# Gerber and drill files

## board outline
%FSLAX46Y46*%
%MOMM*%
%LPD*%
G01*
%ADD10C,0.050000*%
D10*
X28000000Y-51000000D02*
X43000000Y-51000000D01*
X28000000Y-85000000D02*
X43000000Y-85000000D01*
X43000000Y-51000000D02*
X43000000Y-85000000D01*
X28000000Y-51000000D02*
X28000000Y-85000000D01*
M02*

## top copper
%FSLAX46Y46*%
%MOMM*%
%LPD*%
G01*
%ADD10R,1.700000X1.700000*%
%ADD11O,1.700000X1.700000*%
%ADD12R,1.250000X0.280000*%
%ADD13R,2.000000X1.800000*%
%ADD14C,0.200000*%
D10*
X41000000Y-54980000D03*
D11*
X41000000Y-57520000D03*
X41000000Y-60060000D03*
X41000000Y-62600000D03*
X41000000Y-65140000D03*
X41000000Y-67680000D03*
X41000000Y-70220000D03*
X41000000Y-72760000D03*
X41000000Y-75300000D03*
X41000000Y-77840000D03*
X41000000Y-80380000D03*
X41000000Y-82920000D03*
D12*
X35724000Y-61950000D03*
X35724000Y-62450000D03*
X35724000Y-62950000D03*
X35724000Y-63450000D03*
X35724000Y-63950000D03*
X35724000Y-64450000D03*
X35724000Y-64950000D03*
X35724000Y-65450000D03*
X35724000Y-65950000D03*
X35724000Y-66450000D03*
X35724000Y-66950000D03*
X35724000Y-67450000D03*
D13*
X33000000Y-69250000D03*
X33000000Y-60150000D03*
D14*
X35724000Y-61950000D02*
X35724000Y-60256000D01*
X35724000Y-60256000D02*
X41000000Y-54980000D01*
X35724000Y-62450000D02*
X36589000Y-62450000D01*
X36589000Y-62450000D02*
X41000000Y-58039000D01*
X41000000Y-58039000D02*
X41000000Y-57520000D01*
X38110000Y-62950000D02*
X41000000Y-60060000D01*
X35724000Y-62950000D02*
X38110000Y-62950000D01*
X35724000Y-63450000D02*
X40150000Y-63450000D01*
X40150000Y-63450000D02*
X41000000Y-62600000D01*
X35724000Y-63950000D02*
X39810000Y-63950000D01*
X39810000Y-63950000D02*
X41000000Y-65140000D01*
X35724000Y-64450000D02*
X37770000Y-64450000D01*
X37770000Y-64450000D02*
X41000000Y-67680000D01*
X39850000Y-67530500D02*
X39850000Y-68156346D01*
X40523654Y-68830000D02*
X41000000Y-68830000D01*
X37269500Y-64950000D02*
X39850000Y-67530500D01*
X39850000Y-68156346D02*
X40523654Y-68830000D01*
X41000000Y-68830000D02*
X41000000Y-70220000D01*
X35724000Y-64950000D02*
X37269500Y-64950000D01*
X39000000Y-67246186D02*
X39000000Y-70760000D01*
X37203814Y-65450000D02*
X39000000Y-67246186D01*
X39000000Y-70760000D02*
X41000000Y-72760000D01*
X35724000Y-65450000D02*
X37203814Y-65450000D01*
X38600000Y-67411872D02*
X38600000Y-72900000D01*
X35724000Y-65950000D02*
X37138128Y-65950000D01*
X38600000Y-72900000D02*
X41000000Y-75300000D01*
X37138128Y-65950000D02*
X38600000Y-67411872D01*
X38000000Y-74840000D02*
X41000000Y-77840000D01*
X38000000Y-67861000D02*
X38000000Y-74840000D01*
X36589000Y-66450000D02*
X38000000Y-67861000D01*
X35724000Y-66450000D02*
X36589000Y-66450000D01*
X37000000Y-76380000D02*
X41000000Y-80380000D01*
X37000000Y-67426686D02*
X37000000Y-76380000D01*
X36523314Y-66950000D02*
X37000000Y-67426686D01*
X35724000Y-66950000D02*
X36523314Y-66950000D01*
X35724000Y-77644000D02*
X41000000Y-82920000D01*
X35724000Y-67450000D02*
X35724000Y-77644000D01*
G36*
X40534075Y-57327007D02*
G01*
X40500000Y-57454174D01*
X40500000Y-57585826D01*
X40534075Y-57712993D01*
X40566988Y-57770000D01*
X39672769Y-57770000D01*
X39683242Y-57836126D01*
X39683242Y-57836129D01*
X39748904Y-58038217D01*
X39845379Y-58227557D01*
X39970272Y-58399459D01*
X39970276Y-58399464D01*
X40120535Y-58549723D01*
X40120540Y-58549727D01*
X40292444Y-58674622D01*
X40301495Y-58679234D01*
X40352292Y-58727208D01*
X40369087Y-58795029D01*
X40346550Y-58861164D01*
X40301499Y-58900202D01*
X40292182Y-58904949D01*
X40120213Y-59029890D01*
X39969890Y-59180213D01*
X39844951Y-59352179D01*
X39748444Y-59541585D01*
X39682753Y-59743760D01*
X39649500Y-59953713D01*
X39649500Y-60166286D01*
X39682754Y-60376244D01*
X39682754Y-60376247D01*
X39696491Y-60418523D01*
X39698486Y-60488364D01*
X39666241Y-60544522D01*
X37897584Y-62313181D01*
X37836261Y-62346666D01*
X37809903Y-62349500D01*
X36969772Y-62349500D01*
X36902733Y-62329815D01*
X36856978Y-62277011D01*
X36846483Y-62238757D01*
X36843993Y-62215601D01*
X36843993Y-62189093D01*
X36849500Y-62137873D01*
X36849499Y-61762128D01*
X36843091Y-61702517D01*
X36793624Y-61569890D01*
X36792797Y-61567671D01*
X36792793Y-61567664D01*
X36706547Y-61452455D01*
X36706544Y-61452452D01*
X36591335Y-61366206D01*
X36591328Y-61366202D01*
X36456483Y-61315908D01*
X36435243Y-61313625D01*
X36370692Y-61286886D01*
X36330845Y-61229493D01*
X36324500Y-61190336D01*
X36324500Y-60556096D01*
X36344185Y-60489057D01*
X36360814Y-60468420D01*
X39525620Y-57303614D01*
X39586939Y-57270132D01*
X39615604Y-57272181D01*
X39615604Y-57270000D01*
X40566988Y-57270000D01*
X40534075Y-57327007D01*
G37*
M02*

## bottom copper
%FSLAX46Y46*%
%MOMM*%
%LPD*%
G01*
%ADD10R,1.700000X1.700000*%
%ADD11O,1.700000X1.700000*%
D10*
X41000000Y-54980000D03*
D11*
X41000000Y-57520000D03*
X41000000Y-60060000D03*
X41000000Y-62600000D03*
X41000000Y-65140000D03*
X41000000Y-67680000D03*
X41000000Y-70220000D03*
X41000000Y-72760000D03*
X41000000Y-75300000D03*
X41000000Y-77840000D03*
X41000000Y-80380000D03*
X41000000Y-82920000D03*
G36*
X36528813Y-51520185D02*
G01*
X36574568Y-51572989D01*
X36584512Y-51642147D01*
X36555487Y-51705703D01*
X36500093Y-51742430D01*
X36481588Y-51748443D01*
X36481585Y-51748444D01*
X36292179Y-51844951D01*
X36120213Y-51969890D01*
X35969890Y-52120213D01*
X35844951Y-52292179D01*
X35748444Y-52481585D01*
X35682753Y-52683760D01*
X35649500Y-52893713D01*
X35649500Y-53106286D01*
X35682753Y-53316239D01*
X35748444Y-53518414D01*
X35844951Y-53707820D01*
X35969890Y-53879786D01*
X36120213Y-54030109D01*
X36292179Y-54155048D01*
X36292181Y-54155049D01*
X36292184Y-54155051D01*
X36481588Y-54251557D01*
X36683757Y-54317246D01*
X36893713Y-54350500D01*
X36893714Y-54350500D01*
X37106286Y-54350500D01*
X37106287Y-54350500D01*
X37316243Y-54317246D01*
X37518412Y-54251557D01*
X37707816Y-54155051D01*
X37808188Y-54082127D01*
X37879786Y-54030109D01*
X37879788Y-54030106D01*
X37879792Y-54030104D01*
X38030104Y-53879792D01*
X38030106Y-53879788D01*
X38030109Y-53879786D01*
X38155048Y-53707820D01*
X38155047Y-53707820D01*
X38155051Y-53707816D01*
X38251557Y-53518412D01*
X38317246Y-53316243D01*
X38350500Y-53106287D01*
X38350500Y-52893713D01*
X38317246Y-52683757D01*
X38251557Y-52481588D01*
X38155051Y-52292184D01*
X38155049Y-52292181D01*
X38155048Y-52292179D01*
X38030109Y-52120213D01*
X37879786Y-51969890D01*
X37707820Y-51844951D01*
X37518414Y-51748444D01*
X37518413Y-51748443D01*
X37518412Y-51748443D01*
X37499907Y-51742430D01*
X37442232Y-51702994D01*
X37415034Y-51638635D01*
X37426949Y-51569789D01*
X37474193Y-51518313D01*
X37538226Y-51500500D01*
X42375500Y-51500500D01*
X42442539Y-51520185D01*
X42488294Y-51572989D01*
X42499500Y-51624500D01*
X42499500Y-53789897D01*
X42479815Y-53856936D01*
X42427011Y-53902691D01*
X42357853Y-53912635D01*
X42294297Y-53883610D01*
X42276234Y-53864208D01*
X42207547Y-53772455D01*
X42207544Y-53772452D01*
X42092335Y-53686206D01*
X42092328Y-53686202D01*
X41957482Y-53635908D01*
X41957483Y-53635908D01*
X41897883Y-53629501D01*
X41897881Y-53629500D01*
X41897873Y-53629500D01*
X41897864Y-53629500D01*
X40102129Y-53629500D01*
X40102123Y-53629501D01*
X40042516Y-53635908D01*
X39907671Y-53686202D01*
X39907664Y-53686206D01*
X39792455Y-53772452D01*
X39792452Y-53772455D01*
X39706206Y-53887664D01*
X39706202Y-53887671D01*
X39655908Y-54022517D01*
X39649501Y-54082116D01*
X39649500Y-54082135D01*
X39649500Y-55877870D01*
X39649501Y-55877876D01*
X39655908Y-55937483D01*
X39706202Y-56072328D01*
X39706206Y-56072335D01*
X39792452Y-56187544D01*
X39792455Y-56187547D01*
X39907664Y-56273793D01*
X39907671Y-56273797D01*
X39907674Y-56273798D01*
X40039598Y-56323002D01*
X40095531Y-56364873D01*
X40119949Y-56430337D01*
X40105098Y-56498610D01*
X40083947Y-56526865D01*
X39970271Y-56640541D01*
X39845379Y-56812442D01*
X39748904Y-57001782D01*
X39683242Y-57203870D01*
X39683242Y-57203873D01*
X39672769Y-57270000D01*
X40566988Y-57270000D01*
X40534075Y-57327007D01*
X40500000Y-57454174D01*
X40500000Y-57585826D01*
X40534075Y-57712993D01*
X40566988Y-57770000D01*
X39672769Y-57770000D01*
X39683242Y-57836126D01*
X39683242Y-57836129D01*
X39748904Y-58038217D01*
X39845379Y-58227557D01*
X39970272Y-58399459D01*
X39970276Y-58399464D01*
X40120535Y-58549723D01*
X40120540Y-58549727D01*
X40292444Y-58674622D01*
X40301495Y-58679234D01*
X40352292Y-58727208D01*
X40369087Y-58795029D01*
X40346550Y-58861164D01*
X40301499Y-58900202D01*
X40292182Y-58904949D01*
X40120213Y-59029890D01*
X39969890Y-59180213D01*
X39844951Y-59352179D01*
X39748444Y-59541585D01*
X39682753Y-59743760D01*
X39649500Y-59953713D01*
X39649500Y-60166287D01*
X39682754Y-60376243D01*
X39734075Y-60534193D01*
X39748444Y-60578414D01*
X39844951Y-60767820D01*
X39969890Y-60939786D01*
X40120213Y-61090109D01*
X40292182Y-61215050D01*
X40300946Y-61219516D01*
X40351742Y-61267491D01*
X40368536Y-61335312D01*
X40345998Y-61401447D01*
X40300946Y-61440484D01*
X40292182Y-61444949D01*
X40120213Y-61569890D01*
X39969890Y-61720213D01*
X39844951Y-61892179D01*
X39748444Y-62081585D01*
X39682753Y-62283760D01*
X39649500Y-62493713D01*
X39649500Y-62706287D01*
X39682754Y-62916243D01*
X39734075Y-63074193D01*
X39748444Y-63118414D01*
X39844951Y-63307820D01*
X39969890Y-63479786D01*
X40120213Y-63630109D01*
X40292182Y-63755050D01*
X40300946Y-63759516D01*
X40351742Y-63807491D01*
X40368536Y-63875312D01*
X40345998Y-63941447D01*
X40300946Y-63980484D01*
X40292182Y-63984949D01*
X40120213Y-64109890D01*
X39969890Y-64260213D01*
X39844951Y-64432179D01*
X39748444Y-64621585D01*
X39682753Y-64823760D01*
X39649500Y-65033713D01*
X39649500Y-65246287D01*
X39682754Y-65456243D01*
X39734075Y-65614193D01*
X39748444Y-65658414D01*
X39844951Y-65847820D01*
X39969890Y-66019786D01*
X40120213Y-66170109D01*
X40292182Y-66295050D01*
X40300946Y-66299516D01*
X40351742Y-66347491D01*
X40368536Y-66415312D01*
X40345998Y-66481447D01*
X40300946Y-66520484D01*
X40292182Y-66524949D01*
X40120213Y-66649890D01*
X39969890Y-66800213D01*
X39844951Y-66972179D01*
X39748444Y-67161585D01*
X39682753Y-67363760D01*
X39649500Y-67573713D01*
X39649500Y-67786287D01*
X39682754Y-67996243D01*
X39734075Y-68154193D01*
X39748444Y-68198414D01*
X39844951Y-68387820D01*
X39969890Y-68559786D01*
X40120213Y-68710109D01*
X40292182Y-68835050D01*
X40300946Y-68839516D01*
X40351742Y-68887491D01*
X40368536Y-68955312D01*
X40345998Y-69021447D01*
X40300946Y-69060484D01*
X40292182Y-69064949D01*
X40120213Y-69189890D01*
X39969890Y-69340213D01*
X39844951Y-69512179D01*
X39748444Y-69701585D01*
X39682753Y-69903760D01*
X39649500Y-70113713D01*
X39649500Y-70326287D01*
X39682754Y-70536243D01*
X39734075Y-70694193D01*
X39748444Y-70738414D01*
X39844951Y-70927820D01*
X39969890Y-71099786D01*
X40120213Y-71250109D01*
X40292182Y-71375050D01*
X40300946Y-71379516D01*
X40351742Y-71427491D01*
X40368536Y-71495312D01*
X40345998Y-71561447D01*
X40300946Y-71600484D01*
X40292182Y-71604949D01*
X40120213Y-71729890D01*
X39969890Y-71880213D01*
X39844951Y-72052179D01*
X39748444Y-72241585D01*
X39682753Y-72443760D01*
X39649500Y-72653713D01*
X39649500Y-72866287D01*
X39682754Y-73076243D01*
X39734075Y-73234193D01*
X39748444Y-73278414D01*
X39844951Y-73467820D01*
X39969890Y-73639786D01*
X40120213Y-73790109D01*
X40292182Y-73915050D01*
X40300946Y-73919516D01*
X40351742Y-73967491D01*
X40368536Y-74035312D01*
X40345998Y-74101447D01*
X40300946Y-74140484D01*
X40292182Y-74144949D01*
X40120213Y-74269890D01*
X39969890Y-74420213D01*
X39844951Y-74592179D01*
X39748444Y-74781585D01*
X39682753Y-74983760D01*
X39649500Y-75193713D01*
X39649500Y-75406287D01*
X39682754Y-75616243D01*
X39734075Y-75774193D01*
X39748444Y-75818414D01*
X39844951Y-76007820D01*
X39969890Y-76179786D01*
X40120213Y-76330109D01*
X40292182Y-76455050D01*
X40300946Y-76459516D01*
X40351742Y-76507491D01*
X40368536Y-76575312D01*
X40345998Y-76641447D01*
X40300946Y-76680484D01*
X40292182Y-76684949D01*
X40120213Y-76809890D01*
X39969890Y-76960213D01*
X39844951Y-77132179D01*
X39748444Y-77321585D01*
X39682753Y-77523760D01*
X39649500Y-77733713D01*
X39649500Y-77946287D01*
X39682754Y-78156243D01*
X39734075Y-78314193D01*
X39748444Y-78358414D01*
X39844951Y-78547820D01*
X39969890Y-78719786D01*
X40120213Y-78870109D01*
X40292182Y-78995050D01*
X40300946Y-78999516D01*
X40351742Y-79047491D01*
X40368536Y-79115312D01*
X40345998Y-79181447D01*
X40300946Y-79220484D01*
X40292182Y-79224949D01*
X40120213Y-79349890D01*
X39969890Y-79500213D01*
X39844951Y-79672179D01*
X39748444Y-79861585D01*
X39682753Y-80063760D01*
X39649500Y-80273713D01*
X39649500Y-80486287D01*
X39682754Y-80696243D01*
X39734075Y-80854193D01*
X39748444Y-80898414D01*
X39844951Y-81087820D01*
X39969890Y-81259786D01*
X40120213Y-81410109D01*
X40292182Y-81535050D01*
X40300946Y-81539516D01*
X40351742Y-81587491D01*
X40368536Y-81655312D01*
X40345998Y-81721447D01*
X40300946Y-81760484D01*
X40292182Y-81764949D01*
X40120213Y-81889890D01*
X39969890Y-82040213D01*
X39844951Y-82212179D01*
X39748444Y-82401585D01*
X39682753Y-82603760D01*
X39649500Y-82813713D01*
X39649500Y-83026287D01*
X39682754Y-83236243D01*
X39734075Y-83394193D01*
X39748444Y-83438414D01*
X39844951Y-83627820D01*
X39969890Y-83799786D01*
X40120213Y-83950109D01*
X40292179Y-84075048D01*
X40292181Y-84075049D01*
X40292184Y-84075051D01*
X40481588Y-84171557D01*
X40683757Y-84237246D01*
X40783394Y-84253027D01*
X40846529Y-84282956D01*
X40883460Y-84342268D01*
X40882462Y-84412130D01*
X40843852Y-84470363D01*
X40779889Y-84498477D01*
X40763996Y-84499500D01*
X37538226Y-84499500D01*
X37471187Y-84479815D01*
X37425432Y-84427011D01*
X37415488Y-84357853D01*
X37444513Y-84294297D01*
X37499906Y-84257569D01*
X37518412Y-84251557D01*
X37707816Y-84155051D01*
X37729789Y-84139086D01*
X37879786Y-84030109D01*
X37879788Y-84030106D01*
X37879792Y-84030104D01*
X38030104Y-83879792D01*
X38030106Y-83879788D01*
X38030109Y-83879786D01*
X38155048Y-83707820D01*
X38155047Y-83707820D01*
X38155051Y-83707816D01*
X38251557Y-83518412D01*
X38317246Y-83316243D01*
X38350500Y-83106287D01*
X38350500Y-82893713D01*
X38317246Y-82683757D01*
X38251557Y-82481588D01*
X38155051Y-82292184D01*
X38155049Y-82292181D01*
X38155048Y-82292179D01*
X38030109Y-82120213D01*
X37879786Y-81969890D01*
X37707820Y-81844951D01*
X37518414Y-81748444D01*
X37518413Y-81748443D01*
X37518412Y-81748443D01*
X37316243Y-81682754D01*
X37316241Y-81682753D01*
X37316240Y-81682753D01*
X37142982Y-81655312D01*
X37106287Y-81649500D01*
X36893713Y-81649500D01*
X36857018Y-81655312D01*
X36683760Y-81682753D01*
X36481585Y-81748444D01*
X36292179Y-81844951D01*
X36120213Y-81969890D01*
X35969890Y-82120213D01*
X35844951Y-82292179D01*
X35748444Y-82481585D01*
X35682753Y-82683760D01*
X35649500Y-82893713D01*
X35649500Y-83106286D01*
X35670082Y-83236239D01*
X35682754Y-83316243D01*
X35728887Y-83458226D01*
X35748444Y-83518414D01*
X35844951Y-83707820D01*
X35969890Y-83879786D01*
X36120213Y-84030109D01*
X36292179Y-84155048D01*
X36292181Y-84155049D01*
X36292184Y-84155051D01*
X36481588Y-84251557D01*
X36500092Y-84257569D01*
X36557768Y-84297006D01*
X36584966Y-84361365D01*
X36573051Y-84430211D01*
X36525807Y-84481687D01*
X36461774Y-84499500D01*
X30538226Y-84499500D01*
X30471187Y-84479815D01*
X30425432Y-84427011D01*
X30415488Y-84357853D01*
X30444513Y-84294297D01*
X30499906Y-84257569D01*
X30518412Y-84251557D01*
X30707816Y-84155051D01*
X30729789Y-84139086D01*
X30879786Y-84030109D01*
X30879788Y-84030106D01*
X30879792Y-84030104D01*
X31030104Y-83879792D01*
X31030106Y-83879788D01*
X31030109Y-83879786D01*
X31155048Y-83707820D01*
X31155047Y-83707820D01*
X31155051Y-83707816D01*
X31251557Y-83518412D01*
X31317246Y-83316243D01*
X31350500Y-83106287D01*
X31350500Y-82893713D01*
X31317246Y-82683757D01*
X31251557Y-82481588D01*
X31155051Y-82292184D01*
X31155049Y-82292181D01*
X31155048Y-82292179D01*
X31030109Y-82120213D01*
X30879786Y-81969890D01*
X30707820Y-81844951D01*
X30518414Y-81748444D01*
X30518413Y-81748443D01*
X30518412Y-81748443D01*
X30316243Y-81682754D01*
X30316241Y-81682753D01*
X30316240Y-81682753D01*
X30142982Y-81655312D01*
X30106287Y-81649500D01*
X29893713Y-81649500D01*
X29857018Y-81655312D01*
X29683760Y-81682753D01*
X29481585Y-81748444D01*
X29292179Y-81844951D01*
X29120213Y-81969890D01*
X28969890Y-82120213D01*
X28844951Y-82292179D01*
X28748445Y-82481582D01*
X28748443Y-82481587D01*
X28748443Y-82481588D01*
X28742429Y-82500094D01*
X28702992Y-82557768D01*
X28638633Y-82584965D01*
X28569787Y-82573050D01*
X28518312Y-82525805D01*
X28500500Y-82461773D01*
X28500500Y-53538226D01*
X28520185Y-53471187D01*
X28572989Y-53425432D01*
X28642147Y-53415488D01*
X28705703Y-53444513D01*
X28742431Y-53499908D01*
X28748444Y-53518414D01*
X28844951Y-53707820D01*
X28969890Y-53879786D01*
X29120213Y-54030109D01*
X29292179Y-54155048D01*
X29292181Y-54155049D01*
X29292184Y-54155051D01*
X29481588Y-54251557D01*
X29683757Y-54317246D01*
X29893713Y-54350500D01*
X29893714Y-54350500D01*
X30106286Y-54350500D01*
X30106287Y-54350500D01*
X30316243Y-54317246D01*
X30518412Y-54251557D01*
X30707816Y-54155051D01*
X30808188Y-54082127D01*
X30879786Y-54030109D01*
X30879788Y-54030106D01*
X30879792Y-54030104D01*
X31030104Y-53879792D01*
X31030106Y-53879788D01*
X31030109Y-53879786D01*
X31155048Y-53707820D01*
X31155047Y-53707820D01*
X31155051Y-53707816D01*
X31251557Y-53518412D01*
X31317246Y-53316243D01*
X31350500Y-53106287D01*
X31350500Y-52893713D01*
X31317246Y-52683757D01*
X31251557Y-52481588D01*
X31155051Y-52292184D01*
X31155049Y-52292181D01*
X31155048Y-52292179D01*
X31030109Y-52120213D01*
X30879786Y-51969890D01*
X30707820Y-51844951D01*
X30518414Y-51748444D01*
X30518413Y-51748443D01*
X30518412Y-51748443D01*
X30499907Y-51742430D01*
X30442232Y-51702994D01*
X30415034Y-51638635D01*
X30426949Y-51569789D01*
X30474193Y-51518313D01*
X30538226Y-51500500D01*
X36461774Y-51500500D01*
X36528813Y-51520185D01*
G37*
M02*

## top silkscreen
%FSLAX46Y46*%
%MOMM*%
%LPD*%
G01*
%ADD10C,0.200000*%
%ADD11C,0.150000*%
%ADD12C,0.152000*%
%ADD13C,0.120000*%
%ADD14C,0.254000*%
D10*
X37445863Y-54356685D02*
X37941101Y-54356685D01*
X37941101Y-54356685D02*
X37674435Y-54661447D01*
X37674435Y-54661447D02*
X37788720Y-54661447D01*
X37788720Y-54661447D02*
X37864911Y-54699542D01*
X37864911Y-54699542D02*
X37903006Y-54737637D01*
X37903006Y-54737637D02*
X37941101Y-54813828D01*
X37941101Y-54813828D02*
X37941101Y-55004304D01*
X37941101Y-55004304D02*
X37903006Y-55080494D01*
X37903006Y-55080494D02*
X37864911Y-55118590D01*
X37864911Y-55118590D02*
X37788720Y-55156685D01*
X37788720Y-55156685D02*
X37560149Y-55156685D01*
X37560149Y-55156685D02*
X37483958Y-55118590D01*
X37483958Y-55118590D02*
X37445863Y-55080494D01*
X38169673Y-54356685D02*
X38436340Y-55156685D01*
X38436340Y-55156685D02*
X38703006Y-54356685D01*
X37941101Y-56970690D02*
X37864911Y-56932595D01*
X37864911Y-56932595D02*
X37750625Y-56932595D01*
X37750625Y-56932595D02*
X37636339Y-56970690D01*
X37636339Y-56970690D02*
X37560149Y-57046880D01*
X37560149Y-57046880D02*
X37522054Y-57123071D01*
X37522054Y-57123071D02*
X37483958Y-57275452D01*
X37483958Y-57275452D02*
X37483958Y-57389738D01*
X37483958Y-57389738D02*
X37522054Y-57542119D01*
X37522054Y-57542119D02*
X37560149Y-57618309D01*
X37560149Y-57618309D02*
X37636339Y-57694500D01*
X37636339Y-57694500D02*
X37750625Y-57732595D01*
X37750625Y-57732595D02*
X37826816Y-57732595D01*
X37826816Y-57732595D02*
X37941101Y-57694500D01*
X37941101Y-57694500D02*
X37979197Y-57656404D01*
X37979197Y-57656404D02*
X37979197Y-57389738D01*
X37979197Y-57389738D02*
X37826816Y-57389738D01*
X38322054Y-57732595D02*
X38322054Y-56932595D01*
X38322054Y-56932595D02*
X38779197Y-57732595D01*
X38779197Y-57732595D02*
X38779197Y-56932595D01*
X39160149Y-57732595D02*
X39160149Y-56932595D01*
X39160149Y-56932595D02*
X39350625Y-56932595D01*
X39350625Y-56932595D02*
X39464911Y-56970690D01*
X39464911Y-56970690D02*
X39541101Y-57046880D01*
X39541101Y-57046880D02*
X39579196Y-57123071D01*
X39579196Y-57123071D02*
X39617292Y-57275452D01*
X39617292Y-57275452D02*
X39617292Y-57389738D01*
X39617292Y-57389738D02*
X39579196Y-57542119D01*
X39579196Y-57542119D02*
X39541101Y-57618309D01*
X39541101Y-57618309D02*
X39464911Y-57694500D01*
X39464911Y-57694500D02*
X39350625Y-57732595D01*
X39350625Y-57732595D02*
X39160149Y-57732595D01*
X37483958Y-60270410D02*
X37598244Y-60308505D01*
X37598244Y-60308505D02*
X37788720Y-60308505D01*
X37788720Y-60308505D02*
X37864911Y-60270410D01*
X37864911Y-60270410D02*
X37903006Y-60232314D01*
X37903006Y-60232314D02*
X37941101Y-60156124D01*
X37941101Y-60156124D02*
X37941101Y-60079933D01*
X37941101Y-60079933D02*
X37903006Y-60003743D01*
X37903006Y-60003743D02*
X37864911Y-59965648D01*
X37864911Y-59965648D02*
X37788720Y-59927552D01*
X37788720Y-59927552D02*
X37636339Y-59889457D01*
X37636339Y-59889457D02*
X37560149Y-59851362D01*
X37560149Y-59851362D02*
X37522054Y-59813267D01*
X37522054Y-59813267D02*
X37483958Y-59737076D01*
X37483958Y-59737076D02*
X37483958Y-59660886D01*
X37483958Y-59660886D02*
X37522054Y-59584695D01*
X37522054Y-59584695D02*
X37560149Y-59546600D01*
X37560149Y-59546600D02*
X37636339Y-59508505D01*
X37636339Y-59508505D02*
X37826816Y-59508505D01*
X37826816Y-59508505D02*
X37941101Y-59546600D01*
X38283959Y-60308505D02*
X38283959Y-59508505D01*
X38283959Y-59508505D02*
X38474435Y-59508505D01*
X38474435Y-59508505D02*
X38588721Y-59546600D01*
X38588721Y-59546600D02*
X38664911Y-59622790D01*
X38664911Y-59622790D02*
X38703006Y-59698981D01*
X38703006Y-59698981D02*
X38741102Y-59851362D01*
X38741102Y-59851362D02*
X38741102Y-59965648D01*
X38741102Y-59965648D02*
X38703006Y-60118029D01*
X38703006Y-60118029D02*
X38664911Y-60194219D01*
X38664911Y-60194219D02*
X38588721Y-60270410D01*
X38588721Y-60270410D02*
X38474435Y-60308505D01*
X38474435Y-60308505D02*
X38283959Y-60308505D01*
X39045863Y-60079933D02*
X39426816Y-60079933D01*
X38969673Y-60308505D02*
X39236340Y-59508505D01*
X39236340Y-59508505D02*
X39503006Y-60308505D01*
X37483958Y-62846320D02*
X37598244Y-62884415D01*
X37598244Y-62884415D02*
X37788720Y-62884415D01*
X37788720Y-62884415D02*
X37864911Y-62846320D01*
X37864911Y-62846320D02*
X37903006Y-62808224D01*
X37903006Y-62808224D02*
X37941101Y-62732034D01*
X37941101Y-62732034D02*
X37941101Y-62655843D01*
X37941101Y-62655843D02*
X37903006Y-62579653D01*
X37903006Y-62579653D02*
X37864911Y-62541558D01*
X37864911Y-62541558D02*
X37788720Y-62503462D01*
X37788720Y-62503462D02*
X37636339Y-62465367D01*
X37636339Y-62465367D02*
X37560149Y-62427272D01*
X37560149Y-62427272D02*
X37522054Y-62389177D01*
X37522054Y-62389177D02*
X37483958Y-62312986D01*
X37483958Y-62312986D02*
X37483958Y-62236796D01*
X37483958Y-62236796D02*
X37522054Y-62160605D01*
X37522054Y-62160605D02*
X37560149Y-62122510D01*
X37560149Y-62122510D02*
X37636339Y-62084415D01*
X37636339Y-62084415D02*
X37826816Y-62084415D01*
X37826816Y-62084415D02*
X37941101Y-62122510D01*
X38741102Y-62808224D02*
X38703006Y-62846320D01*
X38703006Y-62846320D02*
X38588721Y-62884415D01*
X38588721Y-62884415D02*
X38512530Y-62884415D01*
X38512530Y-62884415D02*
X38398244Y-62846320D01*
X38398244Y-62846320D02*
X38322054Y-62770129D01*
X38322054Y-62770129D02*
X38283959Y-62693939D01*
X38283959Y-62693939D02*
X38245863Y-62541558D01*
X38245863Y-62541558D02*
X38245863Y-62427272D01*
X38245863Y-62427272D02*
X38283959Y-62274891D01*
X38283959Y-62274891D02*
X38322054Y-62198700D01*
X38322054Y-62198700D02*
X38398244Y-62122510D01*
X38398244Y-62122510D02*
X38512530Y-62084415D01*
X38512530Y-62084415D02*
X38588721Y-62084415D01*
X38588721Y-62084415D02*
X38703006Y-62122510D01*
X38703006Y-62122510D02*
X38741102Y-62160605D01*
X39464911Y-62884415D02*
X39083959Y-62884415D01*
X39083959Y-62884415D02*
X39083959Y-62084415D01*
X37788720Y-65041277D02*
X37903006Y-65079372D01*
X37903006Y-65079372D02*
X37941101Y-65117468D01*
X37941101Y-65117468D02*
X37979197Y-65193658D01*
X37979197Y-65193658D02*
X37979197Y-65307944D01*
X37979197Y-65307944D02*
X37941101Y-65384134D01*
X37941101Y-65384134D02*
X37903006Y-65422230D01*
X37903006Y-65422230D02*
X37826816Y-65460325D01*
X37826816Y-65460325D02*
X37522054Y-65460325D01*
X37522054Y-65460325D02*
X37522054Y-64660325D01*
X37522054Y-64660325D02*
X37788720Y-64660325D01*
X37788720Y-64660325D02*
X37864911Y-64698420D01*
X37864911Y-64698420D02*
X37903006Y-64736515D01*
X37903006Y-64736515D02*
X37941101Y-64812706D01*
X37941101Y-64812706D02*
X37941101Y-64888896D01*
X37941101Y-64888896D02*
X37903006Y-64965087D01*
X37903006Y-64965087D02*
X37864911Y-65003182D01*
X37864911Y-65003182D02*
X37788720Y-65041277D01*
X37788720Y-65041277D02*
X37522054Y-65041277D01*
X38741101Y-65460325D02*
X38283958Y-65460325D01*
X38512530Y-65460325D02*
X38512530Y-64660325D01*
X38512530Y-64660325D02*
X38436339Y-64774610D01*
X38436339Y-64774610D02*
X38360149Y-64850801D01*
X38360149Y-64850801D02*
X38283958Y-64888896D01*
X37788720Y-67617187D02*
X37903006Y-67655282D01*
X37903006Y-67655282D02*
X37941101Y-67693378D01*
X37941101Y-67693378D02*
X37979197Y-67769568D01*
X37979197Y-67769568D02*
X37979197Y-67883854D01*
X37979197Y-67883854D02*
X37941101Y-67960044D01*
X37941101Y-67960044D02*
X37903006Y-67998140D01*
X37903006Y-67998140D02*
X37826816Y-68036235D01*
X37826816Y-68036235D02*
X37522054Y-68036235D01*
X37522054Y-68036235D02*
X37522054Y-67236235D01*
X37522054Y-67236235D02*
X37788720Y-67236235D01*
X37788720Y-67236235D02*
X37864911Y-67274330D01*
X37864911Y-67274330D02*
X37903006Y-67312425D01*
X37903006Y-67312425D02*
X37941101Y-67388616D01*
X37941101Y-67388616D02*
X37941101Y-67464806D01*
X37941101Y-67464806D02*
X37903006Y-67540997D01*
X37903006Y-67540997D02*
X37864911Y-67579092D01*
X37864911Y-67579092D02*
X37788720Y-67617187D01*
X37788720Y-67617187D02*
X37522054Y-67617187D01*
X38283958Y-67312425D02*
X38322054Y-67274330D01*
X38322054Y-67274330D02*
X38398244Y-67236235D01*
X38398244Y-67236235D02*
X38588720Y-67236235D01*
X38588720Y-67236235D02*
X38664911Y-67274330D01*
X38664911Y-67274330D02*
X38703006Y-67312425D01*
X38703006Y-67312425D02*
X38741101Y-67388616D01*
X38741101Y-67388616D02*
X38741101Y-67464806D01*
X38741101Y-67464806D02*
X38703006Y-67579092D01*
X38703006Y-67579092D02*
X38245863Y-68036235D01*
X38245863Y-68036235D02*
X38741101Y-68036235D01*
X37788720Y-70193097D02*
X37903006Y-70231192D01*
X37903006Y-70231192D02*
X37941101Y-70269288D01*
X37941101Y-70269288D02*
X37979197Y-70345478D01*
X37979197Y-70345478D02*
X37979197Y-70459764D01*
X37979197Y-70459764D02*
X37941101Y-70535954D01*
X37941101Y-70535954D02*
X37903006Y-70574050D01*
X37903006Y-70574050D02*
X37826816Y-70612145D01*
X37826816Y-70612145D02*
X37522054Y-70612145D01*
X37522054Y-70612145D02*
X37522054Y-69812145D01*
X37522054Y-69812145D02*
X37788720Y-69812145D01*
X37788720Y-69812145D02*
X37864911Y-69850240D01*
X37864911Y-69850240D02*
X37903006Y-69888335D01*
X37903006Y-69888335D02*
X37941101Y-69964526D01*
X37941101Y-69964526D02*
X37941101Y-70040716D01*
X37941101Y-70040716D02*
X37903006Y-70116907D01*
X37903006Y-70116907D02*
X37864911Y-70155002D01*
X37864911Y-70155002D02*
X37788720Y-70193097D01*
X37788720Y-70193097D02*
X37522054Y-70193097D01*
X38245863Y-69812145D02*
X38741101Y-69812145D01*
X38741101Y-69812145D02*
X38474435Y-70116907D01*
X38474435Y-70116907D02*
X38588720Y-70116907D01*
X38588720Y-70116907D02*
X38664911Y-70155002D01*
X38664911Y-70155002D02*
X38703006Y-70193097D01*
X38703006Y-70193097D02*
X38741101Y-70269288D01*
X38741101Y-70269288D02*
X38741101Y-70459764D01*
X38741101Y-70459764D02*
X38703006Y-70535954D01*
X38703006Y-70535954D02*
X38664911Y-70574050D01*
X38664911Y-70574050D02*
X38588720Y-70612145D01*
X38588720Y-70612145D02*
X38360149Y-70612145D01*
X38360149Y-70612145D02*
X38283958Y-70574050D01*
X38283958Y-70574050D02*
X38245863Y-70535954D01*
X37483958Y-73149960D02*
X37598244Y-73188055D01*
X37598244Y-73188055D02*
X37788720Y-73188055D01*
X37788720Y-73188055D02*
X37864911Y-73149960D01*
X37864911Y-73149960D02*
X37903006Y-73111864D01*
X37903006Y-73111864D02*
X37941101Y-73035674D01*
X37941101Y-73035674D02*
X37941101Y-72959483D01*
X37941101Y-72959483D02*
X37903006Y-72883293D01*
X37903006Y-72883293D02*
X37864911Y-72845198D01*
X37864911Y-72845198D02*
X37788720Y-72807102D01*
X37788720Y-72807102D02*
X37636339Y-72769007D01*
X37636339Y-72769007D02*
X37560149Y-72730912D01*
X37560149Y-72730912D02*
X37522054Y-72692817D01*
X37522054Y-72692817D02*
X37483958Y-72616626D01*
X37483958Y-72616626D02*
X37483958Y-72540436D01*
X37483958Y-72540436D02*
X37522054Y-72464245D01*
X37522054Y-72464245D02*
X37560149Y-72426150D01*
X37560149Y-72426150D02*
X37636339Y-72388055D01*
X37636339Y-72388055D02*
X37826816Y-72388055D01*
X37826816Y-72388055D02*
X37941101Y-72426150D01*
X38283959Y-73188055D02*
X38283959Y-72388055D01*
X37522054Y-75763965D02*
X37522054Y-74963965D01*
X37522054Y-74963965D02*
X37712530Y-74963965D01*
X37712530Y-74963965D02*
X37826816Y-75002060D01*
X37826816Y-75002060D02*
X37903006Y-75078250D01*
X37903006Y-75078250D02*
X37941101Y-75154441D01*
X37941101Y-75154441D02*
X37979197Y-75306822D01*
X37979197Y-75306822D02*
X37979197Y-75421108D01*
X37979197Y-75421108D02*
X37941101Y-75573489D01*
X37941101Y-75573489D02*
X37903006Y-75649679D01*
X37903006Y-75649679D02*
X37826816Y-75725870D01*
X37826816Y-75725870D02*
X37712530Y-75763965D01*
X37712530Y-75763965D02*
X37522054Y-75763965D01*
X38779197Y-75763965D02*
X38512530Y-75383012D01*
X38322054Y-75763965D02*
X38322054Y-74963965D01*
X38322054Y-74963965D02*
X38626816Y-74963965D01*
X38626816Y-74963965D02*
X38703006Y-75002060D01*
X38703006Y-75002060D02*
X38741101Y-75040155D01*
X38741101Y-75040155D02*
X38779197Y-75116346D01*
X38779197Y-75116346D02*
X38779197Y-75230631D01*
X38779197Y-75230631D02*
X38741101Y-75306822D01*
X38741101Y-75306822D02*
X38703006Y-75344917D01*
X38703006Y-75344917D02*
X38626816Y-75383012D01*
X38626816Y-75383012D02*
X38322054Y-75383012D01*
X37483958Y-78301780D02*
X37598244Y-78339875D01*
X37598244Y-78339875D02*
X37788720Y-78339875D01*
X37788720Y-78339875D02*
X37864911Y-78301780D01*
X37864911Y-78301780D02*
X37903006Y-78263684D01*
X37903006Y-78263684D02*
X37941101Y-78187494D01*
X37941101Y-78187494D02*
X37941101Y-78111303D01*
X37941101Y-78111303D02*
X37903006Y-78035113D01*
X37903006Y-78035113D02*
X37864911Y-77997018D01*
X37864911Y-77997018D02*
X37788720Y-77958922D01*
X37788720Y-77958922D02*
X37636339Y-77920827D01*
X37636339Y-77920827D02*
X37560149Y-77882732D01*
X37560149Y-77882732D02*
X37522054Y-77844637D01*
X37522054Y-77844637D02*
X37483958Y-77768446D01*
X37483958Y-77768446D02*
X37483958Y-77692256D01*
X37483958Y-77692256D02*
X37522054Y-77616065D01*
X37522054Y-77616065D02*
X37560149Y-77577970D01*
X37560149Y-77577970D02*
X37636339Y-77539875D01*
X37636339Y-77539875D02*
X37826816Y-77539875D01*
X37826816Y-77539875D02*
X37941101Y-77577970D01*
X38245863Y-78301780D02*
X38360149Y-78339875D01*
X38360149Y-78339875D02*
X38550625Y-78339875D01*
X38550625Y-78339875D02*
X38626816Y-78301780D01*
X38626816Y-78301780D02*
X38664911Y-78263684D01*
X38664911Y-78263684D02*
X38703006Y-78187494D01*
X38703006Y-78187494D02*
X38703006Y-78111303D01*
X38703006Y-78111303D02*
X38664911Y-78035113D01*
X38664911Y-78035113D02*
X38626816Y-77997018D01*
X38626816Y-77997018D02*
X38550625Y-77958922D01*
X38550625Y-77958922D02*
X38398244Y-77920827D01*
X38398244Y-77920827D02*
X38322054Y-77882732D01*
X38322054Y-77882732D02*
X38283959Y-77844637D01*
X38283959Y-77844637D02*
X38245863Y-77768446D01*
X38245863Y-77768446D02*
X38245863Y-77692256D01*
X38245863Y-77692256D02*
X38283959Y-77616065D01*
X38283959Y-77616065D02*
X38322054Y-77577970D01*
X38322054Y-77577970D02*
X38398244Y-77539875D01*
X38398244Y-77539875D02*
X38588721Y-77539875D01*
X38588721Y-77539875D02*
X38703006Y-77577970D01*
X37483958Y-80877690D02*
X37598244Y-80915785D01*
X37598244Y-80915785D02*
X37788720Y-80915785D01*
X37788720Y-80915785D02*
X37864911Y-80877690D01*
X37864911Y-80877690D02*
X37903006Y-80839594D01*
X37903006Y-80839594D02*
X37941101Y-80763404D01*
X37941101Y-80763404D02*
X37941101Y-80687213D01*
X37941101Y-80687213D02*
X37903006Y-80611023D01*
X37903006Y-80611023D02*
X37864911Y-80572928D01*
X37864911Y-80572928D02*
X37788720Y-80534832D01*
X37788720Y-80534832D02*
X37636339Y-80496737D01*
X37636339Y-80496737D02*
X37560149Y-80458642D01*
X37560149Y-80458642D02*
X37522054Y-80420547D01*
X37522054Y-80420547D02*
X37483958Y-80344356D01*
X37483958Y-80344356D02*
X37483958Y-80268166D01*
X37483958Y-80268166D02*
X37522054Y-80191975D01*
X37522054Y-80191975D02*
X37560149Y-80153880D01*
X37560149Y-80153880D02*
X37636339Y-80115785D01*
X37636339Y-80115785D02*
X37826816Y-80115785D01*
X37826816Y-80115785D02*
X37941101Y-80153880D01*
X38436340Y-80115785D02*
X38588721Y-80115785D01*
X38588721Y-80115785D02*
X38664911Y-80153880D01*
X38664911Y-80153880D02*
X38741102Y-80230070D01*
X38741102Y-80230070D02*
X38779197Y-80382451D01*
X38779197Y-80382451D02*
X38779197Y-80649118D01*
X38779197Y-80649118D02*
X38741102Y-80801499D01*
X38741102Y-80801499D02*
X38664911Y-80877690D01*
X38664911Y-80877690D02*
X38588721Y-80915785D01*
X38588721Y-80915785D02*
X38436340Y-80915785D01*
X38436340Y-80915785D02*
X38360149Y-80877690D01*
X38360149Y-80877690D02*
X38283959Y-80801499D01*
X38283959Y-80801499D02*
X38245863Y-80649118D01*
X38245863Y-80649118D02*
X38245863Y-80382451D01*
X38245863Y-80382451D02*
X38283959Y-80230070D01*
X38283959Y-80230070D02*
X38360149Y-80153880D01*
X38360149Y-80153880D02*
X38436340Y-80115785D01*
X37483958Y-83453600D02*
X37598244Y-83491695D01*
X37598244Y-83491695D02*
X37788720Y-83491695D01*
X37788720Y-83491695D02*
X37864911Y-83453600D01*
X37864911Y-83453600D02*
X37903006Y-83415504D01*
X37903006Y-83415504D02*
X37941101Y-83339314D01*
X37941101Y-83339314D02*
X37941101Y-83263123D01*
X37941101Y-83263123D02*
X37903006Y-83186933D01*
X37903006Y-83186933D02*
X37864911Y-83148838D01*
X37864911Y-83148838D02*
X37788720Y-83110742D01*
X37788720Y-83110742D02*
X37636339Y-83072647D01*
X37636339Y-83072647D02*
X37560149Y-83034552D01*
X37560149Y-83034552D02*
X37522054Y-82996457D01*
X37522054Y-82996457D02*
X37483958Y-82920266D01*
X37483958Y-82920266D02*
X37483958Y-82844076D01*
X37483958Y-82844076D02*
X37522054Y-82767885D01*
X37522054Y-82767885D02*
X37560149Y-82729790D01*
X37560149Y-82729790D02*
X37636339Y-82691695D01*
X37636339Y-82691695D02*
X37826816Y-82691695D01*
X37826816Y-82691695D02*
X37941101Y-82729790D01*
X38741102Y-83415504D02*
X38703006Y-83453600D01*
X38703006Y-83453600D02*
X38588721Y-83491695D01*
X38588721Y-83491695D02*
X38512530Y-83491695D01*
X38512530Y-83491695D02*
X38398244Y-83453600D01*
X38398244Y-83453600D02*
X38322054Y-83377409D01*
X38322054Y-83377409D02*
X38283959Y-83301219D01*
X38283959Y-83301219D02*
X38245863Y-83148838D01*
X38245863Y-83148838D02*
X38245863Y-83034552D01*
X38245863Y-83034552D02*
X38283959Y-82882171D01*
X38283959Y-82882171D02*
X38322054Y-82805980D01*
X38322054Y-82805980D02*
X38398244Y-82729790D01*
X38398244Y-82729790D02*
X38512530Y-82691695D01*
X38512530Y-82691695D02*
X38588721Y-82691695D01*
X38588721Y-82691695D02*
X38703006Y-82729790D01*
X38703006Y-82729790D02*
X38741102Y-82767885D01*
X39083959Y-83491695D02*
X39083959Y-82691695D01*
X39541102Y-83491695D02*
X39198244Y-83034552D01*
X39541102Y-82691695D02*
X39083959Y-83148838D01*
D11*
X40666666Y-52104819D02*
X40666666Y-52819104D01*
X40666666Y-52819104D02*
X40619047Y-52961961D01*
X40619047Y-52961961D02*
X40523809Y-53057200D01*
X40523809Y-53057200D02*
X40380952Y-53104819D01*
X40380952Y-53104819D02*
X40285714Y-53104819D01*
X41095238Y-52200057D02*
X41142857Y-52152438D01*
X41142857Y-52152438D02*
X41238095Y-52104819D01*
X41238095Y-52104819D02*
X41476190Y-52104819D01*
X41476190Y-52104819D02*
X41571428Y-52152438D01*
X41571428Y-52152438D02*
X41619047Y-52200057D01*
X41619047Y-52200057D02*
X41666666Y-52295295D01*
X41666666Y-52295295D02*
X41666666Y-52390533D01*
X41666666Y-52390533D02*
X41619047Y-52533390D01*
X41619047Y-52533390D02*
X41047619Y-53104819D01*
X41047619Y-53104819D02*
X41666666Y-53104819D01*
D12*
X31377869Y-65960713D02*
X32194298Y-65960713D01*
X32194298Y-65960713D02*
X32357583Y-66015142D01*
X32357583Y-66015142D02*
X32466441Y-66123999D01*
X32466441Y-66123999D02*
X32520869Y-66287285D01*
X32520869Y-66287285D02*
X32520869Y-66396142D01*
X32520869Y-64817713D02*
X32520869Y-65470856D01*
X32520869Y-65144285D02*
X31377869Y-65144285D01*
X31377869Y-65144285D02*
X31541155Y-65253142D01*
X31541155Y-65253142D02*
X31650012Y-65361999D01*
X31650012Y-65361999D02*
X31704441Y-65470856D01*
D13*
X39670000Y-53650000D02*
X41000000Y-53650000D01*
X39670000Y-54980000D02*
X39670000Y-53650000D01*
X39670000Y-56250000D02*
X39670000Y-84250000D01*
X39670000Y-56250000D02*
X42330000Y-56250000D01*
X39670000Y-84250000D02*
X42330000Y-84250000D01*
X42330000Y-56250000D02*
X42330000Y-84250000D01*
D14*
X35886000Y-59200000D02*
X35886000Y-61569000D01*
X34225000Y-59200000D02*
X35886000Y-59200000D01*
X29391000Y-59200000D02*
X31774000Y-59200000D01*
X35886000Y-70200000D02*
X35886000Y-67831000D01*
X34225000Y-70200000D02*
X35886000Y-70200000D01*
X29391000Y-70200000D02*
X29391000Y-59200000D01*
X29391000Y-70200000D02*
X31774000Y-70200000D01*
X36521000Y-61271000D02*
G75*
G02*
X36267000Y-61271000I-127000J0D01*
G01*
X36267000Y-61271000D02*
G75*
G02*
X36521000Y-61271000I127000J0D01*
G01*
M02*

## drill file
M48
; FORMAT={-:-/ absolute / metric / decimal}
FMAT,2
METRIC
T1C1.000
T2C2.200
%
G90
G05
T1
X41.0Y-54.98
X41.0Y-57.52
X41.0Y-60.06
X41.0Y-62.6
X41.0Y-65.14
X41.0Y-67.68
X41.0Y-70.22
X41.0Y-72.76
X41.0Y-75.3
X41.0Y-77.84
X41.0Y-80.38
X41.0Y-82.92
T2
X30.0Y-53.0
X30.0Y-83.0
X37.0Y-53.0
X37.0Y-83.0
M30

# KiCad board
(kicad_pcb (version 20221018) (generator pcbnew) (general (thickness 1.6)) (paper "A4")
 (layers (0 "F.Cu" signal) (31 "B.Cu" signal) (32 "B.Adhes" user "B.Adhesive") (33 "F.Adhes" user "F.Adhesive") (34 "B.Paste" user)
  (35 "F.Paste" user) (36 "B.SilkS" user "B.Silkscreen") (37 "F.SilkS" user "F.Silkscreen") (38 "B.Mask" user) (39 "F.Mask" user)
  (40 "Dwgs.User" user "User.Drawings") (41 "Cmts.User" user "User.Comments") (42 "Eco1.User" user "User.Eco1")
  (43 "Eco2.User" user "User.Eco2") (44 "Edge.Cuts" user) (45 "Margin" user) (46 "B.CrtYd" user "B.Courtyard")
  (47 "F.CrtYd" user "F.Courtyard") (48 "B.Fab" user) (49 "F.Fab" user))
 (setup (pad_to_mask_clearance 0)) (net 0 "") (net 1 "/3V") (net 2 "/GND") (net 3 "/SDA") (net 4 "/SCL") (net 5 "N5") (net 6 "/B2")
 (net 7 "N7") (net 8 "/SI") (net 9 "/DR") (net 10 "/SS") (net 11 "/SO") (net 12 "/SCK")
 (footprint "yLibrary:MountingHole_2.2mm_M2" (layer "F.Cu") (at 37 53)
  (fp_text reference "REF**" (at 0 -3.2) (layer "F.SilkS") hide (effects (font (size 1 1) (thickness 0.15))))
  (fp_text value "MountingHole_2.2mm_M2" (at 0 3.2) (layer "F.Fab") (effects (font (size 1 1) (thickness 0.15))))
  (pad "" np_thru_hole circle (at 0 0) (size 2.2 2.2) (drill 2.2) (layers "*.Cu" "*.Mask")))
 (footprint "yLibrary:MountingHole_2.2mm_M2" (layer "F.Cu") (at 30 83)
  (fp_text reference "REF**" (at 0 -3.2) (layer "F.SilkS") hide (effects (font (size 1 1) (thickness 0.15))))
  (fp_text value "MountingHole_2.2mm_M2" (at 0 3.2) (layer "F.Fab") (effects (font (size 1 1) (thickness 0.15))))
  (pad "" np_thru_hole circle (at 0 0) (size 2.2 2.2) (drill 2.2) (layers "*.Cu" "*.Mask")))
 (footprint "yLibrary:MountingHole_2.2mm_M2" (layer "F.Cu") (at 30 53)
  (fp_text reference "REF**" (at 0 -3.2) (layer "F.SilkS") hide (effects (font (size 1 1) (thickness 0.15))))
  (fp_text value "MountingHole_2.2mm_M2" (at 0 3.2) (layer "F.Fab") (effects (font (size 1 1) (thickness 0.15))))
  (pad "" np_thru_hole circle (at 0 0) (size 2.2 2.2) (drill 2.2) (layers "*.Cu" "*.Mask")))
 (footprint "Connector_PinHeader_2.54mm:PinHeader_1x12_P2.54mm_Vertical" (layer "F.Cu") (at 41 54.98)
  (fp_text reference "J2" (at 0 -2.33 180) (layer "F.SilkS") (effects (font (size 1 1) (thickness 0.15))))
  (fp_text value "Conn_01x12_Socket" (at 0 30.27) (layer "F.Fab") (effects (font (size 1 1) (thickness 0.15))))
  (fp_line (start -1.33 -1.33) (end 0 -1.33) (stroke (width 0.12) (type solid)) (layer "F.SilkS"))
  (fp_line (start -1.33 0) (end -1.33 -1.33) (stroke (width 0.12) (type solid)) (layer "F.SilkS"))
  (fp_line (start -1.33 1.27) (end -1.33 29.27) (stroke (width 0.12) (type solid)) (layer "F.SilkS"))
  (fp_line (start -1.33 1.27) (end 1.33 1.27) (stroke (width 0.12) (type solid)) (layer "F.SilkS"))
  (fp_line (start -1.33 29.27) (end 1.33 29.27) (stroke (width 0.12) (type solid)) (layer "F.SilkS"))
  (fp_line (start 1.33 1.27) (end 1.33 29.27) (stroke (width 0.12) (type solid)) (layer "F.SilkS"))
  (pad "1" thru_hole rect (at 0 0) (size 1.7 1.7) (drill 1) (layers "*.Cu" "*.Mask") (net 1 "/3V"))
  (pad "2" thru_hole oval (at 0 2.54) (size 1.7 1.7) (drill 1) (layers "*.Cu" "*.Mask") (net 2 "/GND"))
  (pad "3" thru_hole oval (at 0 5.08) (size 1.7 1.7) (drill 1) (layers "*.Cu" "*.Mask") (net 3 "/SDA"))
  (pad "4" thru_hole oval (at 0 7.62) (size 1.7 1.7) (drill 1) (layers "*.Cu" "*.Mask") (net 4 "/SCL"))
  (pad "5" thru_hole oval (at 0 10.16) (size 1.7 1.7) (drill 1) (layers "*.Cu" "*.Mask") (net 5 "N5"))
  (pad "6" thru_hole oval (at 0 12.7) (size 1.7 1.7) (drill 1) (layers "*.Cu" "*.Mask") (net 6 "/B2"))
  (pad "7" thru_hole oval (at 0 15.24) (size 1.7 1.7) (drill 1) (layers "*.Cu" "*.Mask") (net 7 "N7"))
  (pad "8" thru_hole oval (at 0 17.78) (size 1.7 1.7) (drill 1) (layers "*.Cu" "*.Mask") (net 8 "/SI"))
  (pad "9" thru_hole oval (at 0 20.32) (size 1.7 1.7) (drill 1) (layers "*.Cu" "*.Mask") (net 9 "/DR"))
  (pad "10" thru_hole oval (at 0 22.86) (size 1.7 1.7) (drill 1) (layers "*.Cu" "*.Mask") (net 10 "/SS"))
  (pad "11" thru_hole oval (at 0 25.4) (size 1.7 1.7) (drill 1) (layers "*.Cu" "*.Mask") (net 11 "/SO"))
  (pad "12" thru_hole oval (at 0 27.94) (size 1.7 1.7) (drill 1) (layers "*.Cu" "*.Mask") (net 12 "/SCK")))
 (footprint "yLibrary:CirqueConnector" (layer "F.Cu") (at 34.362 64.7 -90)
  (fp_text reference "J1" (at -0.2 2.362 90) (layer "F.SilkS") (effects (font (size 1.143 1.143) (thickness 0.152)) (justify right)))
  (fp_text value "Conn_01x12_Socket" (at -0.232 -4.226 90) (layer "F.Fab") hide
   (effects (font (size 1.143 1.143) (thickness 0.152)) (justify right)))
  (fp_line (start -5.5 -1.524) (end -3.131 -1.524) (stroke (width 0.254) (type solid)) (layer "F.SilkS"))
  (fp_line (start -5.5 0.137) (end -5.5 -1.524) (stroke (width 0.254) (type solid)) (layer "F.SilkS"))
  (fp_line (start -5.5 4.971) (end -5.5 2.588) (stroke (width 0.254) (type solid)) (layer "F.SilkS"))
  (fp_line (start 5.5 -1.524) (end 3.131 -1.524) (stroke (width 0.254) (type solid)) (layer "F.SilkS"))
  (fp_line (start 5.5 0.137) (end 5.5 -1.524) (stroke (width 0.254) (type solid)) (layer "F.SilkS"))
  (fp_line (start 5.5 4.971) (end -5.5 4.971) (stroke (width 0.254) (type solid)) (layer "F.SilkS"))
  (fp_line (start 5.5 4.971) (end 5.5 2.588) (stroke (width 0.254) (type solid)) (layer "F.SilkS"))
  (fp_circle (center -3.429 -2.032) (end -3.302 -2.032) (stroke (width 0.254) (type solid)) (fill none) (layer "F.SilkS"))
  (pad "1" smd rect (at -2.75 -1.362 270) (size 0.28 1.25) (layers "F.Cu" "F.Paste" "F.Mask") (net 1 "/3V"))
  (pad "2" smd rect (at -2.25 -1.362 270) (size 0.28 1.25) (layers "F.Cu" "F.Paste" "F.Mask") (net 2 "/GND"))
  (pad "3" smd rect (at -1.75 -1.362 270) (size 0.28 1.25) (layers "F.Cu" "F.Paste" "F.Mask") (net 3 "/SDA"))
  (pad "4" smd rect (at -1.25 -1.362 270) (size 0.28 1.25) (layers "F.Cu" "F.Paste" "F.Mask") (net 4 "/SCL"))
  (pad "5" smd rect (at -0.75 -1.362 270) (size 0.28 1.25) (layers "F.Cu" "F.Paste" "F.Mask") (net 5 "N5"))
  (pad "6" smd rect (at -0.25 -1.362 270) (size 0.28 1.25) (layers "F.Cu" "F.Paste" "F.Mask") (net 6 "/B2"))
  (pad "7" smd rect (at 0.25 -1.362 270) (size 0.28 1.25) (layers "F.Cu" "F.Paste" "F.Mask") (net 7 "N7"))
  (pad "8" smd rect (at 0.75 -1.362 270) (size 0.28 1.25) (layers "F.Cu" "F.Paste" "F.Mask") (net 8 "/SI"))
  (pad "9" smd rect (at 1.25 -1.362 270) (size 0.28 1.25) (layers "F.Cu" "F.Paste" "F.Mask") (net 9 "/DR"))
  (pad "10" smd rect (at 1.75 -1.362 270) (size 0.28 1.25) (layers "F.Cu" "F.Paste" "F.Mask") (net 10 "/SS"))
  (pad "11" smd rect (at 2.25 -1.362 270) (size 0.28 1.25) (layers "F.Cu" "F.Paste" "F.Mask") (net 11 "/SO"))
  (pad "12" smd rect (at 2.75 -1.362 270) (size 0.28 1.25) (layers "F.Cu" "F.Paste" "F.Mask") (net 12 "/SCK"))
  (pad "13" smd rect (at 4.55 1.362 270) (size 1.8 2) (layers "F.Cu" "F.Paste" "F.Mask"))
  (pad "14" smd rect (at -4.55 1.362 270) (size 1.8 2) (layers "F.Cu" "F.Paste" "F.Mask")))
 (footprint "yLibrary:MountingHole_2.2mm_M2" (layer "F.Cu") (at 37 83)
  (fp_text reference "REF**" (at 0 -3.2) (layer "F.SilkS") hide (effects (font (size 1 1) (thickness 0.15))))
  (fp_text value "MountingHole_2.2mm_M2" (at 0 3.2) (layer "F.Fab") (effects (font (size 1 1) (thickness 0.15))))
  (pad "" np_thru_hole circle (at 0 0) (size 2.2 2.2) (drill 2.2) (layers "*.Cu" "*.Mask")))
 (gr_line (start 28 51) (end 43 51) (stroke (width 0.05) (type default)) (layer "Edge.Cuts"))
 (gr_line (start 28 85) (end 43 85) (stroke (width 0.05) (type default)) (layer "Edge.Cuts"))
 (gr_line (start 43 51) (end 43 85) (stroke (width 0.05) (type default)) (layer "Edge.Cuts"))
 (gr_line (start 28 51) (end 28 85) (stroke (width 0.05) (type default)) (layer "Edge.Cuts"))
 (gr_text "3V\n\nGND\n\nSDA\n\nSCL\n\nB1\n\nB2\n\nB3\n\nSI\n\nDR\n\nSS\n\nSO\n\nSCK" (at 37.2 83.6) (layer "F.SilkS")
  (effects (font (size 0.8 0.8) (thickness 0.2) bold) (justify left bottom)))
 (segment (start 35.724 61.95) (end 35.724 60.256) (width 0.2) (layer "F.Cu") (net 1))
 (segment (start 35.724 60.256) (end 41 54.98) (width 0.2) (layer "F.Cu") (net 1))
 (segment (start 35.724 62.45) (end 36.589 62.45) (width 0.2) (layer "F.Cu") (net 2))
 (segment (start 36.589 62.45) (end 41 58.039) (width 0.2) (layer "F.Cu") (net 2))
 (segment (start 41 58.039) (end 41 57.52) (width 0.2) (layer "F.Cu") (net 2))
 (segment (start 38.11 62.95) (end 41 60.06) (width 0.2) (layer "F.Cu") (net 3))
 (segment (start 35.724 62.95) (end 38.11 62.95) (width 0.2) (layer "F.Cu") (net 3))
 (segment (start 35.724 63.45) (end 40.15 63.45) (width 0.2) (layer "F.Cu") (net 4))
 (segment (start 40.15 63.45) (end 41 62.6) (width 0.2) (layer "F.Cu") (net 4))
 (segment (start 35.724 63.95) (end 39.81 63.95) (width 0.2) (layer "F.Cu") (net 5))
 (segment (start 39.81 63.95) (end 41 65.14) (width 0.2) (layer "F.Cu") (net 5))
 (segment (start 35.724 64.45) (end 37.77 64.45) (width 0.2) (layer "F.Cu") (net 6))
 (segment (start 37.77 64.45) (end 41 67.68) (width 0.2) (layer "F.Cu") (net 6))
 (segment (start 39.85 67.5305) (end 39.85 68.156346) (width 0.2) (layer "F.Cu") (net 7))
 (segment (start 40.523654 68.83) (end 41 68.83) (width 0.2) (layer "F.Cu") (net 7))
 (segment (start 37.2695 64.95) (end 39.85 67.5305) (width 0.2) (layer "F.Cu") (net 7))
 (segment (start 39.85 68.156346) (end 40.523654 68.83) (width 0.2) (layer "F.Cu") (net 7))
 (segment (start 41 68.83) (end 41 70.22) (width 0.2) (layer "F.Cu") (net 7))
 (segment (start 35.724 64.95) (end 37.2695 64.95) (width 0.2) (layer "F.Cu") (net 7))
 (segment (start 39 67.246186) (end 39 70.76) (width 0.2) (layer "F.Cu") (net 8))
 (segment (start 37.203814 65.45) (end 39 67.246186) (width 0.2) (layer "F.Cu") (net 8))
 (segment (start 39 70.76) (end 41 72.76) (width 0.2) (layer "F.Cu") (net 8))
 (segment (start 35.724 65.45) (end 37.203814 65.45) (width 0.2) (layer "F.Cu") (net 8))
 (segment (start 38.6 67.411872) (end 38.6 72.9) (width 0.2) (layer "F.Cu") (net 9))
 (segment (start 35.724 65.95) (end 37.138128 65.95) (width 0.2) (layer "F.Cu") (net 9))
 (segment (start 38.6 72.9) (end 41 75.3) (width 0.2) (layer "F.Cu") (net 9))
 (segment (start 37.138128 65.95) (end 38.6 67.411872) (width 0.2) (layer "F.Cu") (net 9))
 (segment (start 38 74.84) (end 41 77.84) (width 0.2) (layer "F.Cu") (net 10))
 (segment (start 38 67.861) (end 38 74.84) (width 0.2) (layer "F.Cu") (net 10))
 (segment (start 36.589 66.45) (end 38 67.861) (width 0.2) (layer "F.Cu") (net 10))
 (segment (start 35.724 66.45) (end 36.589 66.45) (width 0.2) (layer "F.Cu") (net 10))
 (segment (start 37 76.38) (end 41 80.38) (width 0.2) (layer "F.Cu") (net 11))
 (segment (start 37 67.426686) (end 37 76.38) (width 0.2) (layer "F.Cu") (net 11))
 (segment (start 36.523314 66.95) (end 37 67.426686) (width 0.2) (layer "F.Cu") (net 11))
 (segment (start 35.724 66.95) (end 36.523314 66.95) (width 0.2) (layer "F.Cu") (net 11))
 (segment (start 35.724 77.644) (end 41 82.92) (width 0.2) (layer "F.Cu") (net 12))
 (segment (start 35.724 67.45) (end 35.724 77.644) (width 0.2) (layer "F.Cu") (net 12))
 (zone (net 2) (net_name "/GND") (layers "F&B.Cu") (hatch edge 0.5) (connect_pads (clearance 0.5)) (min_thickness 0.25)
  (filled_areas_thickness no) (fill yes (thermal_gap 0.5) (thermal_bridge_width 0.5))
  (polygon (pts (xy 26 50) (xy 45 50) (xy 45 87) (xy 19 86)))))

